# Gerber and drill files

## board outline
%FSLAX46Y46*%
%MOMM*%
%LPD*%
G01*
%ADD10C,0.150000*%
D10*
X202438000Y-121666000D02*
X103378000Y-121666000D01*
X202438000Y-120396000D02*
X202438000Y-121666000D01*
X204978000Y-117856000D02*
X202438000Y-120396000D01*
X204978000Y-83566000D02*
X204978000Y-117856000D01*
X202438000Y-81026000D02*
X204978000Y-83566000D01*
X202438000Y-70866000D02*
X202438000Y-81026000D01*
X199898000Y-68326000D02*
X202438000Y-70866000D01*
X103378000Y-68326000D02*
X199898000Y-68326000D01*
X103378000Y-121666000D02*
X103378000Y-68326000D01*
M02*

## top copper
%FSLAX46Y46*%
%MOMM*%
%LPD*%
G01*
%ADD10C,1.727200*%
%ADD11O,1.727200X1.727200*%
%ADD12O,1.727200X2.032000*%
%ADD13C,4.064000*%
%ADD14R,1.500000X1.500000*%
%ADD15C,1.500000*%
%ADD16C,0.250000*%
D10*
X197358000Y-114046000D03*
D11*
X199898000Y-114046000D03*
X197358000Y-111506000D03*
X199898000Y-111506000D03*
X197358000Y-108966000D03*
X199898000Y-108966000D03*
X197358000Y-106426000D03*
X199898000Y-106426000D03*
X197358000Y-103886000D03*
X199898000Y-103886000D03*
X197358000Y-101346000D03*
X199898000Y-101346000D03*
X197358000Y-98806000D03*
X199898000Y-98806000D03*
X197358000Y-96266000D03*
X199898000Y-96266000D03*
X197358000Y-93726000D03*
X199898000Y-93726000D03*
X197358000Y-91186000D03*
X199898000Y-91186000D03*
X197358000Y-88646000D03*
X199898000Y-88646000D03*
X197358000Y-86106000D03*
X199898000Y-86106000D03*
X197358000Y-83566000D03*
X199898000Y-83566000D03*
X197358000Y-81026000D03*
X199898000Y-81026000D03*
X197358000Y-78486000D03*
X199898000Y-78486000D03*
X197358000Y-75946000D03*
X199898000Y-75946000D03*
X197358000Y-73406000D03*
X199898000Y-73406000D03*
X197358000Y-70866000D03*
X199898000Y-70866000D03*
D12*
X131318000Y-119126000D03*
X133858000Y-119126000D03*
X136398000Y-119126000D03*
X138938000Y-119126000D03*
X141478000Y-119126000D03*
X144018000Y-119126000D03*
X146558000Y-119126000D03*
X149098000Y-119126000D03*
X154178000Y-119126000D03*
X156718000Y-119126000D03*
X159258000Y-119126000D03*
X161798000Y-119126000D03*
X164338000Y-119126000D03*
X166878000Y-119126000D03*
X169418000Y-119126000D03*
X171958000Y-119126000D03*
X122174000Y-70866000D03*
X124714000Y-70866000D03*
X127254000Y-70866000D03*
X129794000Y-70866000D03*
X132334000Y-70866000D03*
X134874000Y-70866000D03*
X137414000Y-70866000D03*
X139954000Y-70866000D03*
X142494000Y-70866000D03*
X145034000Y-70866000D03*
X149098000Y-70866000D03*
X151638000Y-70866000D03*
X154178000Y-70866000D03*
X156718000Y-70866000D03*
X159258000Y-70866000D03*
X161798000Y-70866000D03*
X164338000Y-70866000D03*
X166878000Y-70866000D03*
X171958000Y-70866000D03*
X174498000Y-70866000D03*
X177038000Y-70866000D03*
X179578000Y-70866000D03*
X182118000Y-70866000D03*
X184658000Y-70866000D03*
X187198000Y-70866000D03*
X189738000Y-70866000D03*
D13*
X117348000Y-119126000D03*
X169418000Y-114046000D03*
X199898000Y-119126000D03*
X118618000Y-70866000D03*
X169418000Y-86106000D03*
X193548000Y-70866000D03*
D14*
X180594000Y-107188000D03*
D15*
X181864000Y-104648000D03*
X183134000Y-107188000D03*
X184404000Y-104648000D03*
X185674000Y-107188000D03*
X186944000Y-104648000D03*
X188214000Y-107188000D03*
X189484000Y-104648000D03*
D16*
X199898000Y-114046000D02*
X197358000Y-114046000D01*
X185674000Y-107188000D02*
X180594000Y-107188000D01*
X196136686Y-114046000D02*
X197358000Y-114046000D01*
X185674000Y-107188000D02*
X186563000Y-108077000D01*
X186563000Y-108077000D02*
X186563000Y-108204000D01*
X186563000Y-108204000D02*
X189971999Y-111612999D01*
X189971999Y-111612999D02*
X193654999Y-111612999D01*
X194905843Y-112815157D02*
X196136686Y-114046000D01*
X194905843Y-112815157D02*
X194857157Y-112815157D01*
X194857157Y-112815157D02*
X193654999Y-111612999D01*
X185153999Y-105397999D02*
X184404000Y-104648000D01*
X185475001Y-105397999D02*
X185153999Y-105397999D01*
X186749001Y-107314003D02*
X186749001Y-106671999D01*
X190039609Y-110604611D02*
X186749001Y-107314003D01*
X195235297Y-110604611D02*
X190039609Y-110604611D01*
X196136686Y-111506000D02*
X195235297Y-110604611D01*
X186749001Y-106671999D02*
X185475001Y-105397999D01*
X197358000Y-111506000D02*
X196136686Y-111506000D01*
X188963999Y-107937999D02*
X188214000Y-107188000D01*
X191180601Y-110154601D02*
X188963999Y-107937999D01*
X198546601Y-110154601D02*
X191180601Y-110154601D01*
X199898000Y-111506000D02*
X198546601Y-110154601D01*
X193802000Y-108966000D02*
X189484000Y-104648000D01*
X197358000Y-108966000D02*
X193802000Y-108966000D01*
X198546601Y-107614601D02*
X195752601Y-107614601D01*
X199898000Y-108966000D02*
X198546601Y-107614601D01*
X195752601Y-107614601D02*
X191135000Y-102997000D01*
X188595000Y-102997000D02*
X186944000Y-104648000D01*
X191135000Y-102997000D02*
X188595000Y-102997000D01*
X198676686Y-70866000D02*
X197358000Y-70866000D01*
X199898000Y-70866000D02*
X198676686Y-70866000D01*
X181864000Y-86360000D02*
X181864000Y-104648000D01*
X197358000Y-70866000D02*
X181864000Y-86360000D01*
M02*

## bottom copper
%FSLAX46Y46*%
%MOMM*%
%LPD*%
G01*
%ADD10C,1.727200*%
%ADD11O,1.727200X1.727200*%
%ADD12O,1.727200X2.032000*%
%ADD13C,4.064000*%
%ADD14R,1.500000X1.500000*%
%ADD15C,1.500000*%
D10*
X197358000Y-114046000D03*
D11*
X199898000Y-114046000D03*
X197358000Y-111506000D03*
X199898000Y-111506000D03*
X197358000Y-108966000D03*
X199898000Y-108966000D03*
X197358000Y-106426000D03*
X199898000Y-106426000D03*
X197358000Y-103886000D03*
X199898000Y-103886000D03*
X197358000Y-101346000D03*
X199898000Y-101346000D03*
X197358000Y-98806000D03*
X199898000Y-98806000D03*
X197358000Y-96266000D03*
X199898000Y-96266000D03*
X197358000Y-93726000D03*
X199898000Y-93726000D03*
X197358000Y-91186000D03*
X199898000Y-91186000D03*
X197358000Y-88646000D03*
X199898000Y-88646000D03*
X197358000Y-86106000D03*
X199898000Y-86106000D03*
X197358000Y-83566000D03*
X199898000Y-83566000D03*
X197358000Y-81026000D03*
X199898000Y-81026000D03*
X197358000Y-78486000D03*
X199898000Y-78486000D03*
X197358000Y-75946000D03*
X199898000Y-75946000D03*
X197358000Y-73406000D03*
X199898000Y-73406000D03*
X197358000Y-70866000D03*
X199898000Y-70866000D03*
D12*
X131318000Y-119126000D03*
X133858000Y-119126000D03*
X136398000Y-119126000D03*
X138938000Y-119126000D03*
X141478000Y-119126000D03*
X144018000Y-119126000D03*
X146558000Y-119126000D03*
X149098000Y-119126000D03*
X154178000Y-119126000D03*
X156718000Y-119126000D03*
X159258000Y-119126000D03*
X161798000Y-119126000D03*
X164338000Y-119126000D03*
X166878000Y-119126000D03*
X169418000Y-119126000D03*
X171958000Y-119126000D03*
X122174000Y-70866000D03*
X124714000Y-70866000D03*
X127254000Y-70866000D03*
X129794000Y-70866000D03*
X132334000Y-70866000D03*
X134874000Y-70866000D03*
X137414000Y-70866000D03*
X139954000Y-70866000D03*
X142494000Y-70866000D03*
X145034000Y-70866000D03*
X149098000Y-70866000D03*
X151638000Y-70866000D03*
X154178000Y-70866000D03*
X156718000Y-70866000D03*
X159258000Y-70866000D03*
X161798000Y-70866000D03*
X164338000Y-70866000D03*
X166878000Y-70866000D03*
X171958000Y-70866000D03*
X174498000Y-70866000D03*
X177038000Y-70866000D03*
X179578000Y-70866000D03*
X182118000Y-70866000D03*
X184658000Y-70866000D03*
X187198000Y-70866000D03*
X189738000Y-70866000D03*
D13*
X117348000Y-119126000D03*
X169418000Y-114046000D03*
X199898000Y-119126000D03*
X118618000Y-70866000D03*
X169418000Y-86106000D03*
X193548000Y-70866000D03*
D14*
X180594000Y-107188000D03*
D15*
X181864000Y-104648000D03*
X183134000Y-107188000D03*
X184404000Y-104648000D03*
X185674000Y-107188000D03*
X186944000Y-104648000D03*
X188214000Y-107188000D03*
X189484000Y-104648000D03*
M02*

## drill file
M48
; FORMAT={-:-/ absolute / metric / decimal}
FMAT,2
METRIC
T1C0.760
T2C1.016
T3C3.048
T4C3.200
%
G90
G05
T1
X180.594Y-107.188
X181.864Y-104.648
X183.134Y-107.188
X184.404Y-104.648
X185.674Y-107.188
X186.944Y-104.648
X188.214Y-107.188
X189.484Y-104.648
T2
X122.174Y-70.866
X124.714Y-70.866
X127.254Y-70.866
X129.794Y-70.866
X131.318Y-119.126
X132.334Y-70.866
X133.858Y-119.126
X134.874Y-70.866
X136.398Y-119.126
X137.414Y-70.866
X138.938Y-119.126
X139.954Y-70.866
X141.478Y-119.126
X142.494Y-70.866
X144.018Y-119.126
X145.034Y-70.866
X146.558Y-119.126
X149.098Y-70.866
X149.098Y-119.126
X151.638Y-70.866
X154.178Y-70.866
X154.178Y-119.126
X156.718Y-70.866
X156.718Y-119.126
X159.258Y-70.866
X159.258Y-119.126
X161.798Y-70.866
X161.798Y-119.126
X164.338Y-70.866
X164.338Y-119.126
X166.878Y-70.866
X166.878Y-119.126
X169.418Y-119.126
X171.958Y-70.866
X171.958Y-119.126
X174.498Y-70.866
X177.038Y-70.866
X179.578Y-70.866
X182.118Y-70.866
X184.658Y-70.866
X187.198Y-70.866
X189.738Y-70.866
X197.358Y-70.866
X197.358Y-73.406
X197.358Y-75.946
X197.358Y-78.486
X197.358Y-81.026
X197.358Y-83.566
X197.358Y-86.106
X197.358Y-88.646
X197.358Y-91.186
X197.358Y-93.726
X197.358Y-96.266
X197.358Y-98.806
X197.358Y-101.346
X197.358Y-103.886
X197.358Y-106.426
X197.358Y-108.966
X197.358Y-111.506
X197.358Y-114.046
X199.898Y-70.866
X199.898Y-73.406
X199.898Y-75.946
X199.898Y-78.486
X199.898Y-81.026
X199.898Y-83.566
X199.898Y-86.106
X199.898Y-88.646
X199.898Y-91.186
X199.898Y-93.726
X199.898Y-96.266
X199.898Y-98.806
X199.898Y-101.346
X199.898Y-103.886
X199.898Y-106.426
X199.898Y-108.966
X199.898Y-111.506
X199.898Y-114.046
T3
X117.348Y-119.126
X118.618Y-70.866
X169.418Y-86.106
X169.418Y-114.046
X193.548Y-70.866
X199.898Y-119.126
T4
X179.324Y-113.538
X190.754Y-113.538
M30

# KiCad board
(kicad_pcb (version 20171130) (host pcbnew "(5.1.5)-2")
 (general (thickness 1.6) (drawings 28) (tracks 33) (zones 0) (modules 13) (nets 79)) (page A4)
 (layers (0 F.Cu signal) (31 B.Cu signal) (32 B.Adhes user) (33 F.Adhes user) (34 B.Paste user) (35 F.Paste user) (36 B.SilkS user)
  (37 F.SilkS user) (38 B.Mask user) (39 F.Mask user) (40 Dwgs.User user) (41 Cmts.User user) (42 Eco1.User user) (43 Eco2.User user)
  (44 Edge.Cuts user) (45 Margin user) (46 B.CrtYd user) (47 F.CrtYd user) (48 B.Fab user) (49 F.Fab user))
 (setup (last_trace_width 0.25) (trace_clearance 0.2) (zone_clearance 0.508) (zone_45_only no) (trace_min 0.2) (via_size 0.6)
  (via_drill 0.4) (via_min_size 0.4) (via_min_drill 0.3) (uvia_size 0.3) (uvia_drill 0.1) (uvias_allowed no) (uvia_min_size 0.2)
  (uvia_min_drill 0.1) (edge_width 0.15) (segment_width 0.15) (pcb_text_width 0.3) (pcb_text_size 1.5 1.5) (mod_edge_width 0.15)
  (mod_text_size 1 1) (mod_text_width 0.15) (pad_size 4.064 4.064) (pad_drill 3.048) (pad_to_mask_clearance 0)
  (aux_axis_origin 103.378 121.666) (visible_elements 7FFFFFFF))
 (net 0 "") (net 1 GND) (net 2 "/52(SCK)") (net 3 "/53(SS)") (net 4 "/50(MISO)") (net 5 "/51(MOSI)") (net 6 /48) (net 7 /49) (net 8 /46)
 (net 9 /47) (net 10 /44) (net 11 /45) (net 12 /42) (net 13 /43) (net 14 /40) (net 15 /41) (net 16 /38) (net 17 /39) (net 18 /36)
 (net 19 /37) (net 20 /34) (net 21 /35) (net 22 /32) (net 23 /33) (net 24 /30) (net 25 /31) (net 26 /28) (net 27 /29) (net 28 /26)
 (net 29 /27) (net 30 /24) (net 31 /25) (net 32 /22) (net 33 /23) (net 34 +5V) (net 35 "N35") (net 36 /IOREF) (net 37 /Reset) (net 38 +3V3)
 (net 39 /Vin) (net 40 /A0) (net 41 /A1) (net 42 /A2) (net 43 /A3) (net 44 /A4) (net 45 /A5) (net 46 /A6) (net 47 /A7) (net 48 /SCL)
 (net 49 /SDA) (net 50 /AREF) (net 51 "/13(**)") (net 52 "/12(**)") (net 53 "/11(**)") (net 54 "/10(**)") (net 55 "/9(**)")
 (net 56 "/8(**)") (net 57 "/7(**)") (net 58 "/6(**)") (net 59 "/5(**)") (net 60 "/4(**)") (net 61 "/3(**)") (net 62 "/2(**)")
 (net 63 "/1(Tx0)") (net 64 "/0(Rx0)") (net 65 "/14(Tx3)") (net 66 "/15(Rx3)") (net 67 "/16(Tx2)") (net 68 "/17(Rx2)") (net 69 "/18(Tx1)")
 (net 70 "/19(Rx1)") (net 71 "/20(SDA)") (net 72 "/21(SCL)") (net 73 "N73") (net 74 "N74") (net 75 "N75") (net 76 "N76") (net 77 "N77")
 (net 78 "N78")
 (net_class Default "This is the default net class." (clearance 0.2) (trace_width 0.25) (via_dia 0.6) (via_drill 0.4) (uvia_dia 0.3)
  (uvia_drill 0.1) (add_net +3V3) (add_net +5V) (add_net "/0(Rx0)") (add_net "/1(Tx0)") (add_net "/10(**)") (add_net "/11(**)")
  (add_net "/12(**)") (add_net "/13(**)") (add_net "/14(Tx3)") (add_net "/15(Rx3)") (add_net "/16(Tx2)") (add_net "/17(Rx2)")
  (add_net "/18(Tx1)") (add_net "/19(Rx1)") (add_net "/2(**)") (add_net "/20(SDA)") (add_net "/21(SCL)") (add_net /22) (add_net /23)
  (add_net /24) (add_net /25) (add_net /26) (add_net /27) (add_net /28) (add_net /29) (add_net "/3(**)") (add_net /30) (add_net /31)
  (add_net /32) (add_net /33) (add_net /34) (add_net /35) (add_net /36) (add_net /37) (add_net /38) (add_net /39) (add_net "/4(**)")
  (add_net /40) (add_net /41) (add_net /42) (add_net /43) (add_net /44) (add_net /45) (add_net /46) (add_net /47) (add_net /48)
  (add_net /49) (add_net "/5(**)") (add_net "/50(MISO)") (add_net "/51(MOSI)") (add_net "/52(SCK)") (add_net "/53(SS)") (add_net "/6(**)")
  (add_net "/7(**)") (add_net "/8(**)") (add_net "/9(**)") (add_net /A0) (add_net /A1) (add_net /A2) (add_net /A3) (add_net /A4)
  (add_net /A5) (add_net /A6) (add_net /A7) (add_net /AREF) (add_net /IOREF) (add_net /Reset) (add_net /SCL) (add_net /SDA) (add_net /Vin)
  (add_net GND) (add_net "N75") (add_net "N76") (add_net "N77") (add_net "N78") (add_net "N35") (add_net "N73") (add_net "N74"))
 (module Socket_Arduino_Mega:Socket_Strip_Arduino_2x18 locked (layer F.Cu) (at 197.358 114.046 90)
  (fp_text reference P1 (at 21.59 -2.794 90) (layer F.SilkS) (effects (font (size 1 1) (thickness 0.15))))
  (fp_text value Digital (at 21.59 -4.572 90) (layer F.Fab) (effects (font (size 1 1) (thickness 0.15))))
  (pad 1 thru_hole circle (at 0 0 90) (size 1.7272 1.7272) (drill 1.016) (layers *.Cu *.Mask F.SilkS) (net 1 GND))
  (pad 2 thru_hole oval (at 0 2.54 90) (size 1.7272 1.7272) (drill 1.016) (layers *.Cu *.Mask F.SilkS) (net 1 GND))
  (pad 3 thru_hole oval (at 2.54 0 90) (size 1.7272 1.7272) (drill 1.016) (layers *.Cu *.Mask F.SilkS) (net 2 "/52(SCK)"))
  (pad 4 thru_hole oval (at 2.54 2.54 90) (size 1.7272 1.7272) (drill 1.016) (layers *.Cu *.Mask F.SilkS) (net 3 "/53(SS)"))
  (pad 5 thru_hole oval (at 5.08 0 90) (size 1.7272 1.7272) (drill 1.016) (layers *.Cu *.Mask F.SilkS) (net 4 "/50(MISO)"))
  (pad 6 thru_hole oval (at 5.08 2.54 90) (size 1.7272 1.7272) (drill 1.016) (layers *.Cu *.Mask F.SilkS) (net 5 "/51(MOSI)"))
  (pad 7 thru_hole oval (at 7.62 0 90) (size 1.7272 1.7272) (drill 1.016) (layers *.Cu *.Mask F.SilkS) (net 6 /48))
  (pad 8 thru_hole oval (at 7.62 2.54 90) (size 1.7272 1.7272) (drill 1.016) (layers *.Cu *.Mask F.SilkS) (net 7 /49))
  (pad 9 thru_hole oval (at 10.16 0 90) (size 1.7272 1.7272) (drill 1.016) (layers *.Cu *.Mask F.SilkS) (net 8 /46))
  (pad 10 thru_hole oval (at 10.16 2.54 90) (size 1.7272 1.7272) (drill 1.016) (layers *.Cu *.Mask F.SilkS) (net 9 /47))
  (pad 11 thru_hole oval (at 12.7 0 90) (size 1.7272 1.7272) (drill 1.016) (layers *.Cu *.Mask F.SilkS) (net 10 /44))
  (pad 12 thru_hole oval (at 12.7 2.54 90) (size 1.7272 1.7272) (drill 1.016) (layers *.Cu *.Mask F.SilkS) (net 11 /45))
  (pad 13 thru_hole oval (at 15.24 0 90) (size 1.7272 1.7272) (drill 1.016) (layers *.Cu *.Mask F.SilkS) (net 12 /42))
  (pad 14 thru_hole oval (at 15.24 2.54 90) (size 1.7272 1.7272) (drill 1.016) (layers *.Cu *.Mask F.SilkS) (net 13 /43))
  (pad 15 thru_hole oval (at 17.78 0 90) (size 1.7272 1.7272) (drill 1.016) (layers *.Cu *.Mask F.SilkS) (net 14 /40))
  (pad 16 thru_hole oval (at 17.78 2.54 90) (size 1.7272 1.7272) (drill 1.016) (layers *.Cu *.Mask F.SilkS) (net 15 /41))
  (pad 17 thru_hole oval (at 20.32 0 90) (size 1.7272 1.7272) (drill 1.016) (layers *.Cu *.Mask F.SilkS) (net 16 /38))
  (pad 18 thru_hole oval (at 20.32 2.54 90) (size 1.7272 1.7272) (drill 1.016) (layers *.Cu *.Mask F.SilkS) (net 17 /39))
  (pad 19 thru_hole oval (at 22.86 0 90) (size 1.7272 1.7272) (drill 1.016) (layers *.Cu *.Mask F.SilkS) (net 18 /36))
  (pad 20 thru_hole oval (at 22.86 2.54 90) (size 1.7272 1.7272) (drill 1.016) (layers *.Cu *.Mask F.SilkS) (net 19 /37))
  (pad 21 thru_hole oval (at 25.4 0 90) (size 1.7272 1.7272) (drill 1.016) (layers *.Cu *.Mask F.SilkS) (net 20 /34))
  (pad 22 thru_hole oval (at 25.4 2.54 90) (size 1.7272 1.7272) (drill 1.016) (layers *.Cu *.Mask F.SilkS) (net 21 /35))
  (pad 23 thru_hole oval (at 27.94 0 90) (size 1.7272 1.7272) (drill 1.016) (layers *.Cu *.Mask F.SilkS) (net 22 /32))
  (pad 24 thru_hole oval (at 27.94 2.54 90) (size 1.7272 1.7272) (drill 1.016) (layers *.Cu *.Mask F.SilkS) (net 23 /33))
  (pad 25 thru_hole oval (at 30.48 0 90) (size 1.7272 1.7272) (drill 1.016) (layers *.Cu *.Mask F.SilkS) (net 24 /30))
  (pad 26 thru_hole oval (at 30.48 2.54 90) (size 1.7272 1.7272) (drill 1.016) (layers *.Cu *.Mask F.SilkS) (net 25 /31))
  (pad 27 thru_hole oval (at 33.02 0 90) (size 1.7272 1.7272) (drill 1.016) (layers *.Cu *.Mask F.SilkS) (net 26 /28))
  (pad 28 thru_hole oval (at 33.02 2.54 90) (size 1.7272 1.7272) (drill 1.016) (layers *.Cu *.Mask F.SilkS) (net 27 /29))
  (pad 29 thru_hole oval (at 35.56 0 90) (size 1.7272 1.7272) (drill 1.016) (layers *.Cu *.Mask F.SilkS) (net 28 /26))
  (pad 30 thru_hole oval (at 35.56 2.54 90) (size 1.7272 1.7272) (drill 1.016) (layers *.Cu *.Mask F.SilkS) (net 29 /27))
  (pad 31 thru_hole oval (at 38.1 0 90) (size 1.7272 1.7272) (drill 1.016) (layers *.Cu *.Mask F.SilkS) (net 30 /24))
  (pad 32 thru_hole oval (at 38.1 2.54 90) (size 1.7272 1.7272) (drill 1.016) (layers *.Cu *.Mask F.SilkS) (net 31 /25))
  (pad 33 thru_hole oval (at 40.64 0 90) (size 1.7272 1.7272) (drill 1.016) (layers *.Cu *.Mask F.SilkS) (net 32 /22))
  (pad 34 thru_hole oval (at 40.64 2.54 90) (size 1.7272 1.7272) (drill 1.016) (layers *.Cu *.Mask F.SilkS) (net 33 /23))
  (pad 35 thru_hole oval (at 43.18 0 90) (size 1.7272 1.7272) (drill 1.016) (layers *.Cu *.Mask F.SilkS) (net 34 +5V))
  (pad 36 thru_hole oval (at 43.18 2.54 90) (size 1.7272 1.7272) (drill 1.016) (layers *.Cu *.Mask F.SilkS) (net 34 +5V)))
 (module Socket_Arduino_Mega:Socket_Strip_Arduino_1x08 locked (layer F.Cu) (at 131.318 119.126)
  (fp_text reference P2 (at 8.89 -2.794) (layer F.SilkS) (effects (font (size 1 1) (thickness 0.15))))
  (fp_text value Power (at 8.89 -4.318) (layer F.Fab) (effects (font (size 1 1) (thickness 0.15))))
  (pad 1 thru_hole oval (at 0 0) (size 1.7272 2.032) (drill 1.016) (layers *.Cu *.Mask F.SilkS) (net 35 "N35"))
  (pad 2 thru_hole oval (at 2.54 0) (size 1.7272 2.032) (drill 1.016) (layers *.Cu *.Mask F.SilkS) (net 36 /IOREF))
  (pad 3 thru_hole oval (at 5.08 0) (size 1.7272 2.032) (drill 1.016) (layers *.Cu *.Mask F.SilkS) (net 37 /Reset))
  (pad 4 thru_hole oval (at 7.62 0) (size 1.7272 2.032) (drill 1.016) (layers *.Cu *.Mask F.SilkS) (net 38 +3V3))
  (pad 5 thru_hole oval (at 10.16 0) (size 1.7272 2.032) (drill 1.016) (layers *.Cu *.Mask F.SilkS) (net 34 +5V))
  (pad 6 thru_hole oval (at 12.7 0) (size 1.7272 2.032) (drill 1.016) (layers *.Cu *.Mask F.SilkS) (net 1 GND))
  (pad 7 thru_hole oval (at 15.24 0) (size 1.7272 2.032) (drill 1.016) (layers *.Cu *.Mask F.SilkS) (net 1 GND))
  (pad 8 thru_hole oval (at 17.78 0) (size 1.7272 2.032) (drill 1.016) (layers *.Cu *.Mask F.SilkS) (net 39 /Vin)))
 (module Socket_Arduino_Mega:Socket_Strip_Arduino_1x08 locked (layer F.Cu) (at 154.178 119.126)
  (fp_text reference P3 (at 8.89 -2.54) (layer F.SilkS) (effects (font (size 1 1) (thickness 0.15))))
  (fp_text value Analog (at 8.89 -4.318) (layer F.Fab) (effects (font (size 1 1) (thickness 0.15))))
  (pad 1 thru_hole oval (at 0 0) (size 1.7272 2.032) (drill 1.016) (layers *.Cu *.Mask F.SilkS) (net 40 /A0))
  (pad 2 thru_hole oval (at 2.54 0) (size 1.7272 2.032) (drill 1.016) (layers *.Cu *.Mask F.SilkS) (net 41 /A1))
  (pad 3 thru_hole oval (at 5.08 0) (size 1.7272 2.032) (drill 1.016) (layers *.Cu *.Mask F.SilkS) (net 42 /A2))
  (pad 4 thru_hole oval (at 7.62 0) (size 1.7272 2.032) (drill 1.016) (layers *.Cu *.Mask F.SilkS) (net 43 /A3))
  (pad 5 thru_hole oval (at 10.16 0) (size 1.7272 2.032) (drill 1.016) (layers *.Cu *.Mask F.SilkS) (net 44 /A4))
  (pad 6 thru_hole oval (at 12.7 0) (size 1.7272 2.032) (drill 1.016) (layers *.Cu *.Mask F.SilkS) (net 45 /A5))
  (pad 7 thru_hole oval (at 15.24 0) (size 1.7272 2.032) (drill 1.016) (layers *.Cu *.Mask F.SilkS) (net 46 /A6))
  (pad 8 thru_hole oval (at 17.78 0) (size 1.7272 2.032) (drill 1.016) (layers *.Cu *.Mask F.SilkS) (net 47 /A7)))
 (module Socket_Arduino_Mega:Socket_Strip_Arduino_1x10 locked (layer F.Cu) (at 122.174 70.866)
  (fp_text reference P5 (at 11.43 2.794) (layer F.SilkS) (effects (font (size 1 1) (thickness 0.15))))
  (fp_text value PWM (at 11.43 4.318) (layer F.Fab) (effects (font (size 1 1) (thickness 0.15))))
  (pad 1 thru_hole oval (at 0 0) (size 1.7272 2.032) (drill 1.016) (layers *.Cu *.Mask F.SilkS) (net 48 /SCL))
  (pad 2 thru_hole oval (at 2.54 0) (size 1.7272 2.032) (drill 1.016) (layers *.Cu *.Mask F.SilkS) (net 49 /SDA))
  (pad 3 thru_hole oval (at 5.08 0) (size 1.7272 2.032) (drill 1.016) (layers *.Cu *.Mask F.SilkS) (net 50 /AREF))
  (pad 4 thru_hole oval (at 7.62 0) (size 1.7272 2.032) (drill 1.016) (layers *.Cu *.Mask F.SilkS) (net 1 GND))
  (pad 5 thru_hole oval (at 10.16 0) (size 1.7272 2.032) (drill 1.016) (layers *.Cu *.Mask F.SilkS) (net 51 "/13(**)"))
  (pad 6 thru_hole oval (at 12.7 0) (size 1.7272 2.032) (drill 1.016) (layers *.Cu *.Mask F.SilkS) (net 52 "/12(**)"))
  (pad 7 thru_hole oval (at 15.24 0) (size 1.7272 2.032) (drill 1.016) (layers *.Cu *.Mask F.SilkS) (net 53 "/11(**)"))
  (pad 8 thru_hole oval (at 17.78 0) (size 1.7272 2.032) (drill 1.016) (layers *.Cu *.Mask F.SilkS) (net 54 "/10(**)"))
  (pad 9 thru_hole oval (at 20.32 0) (size 1.7272 2.032) (drill 1.016) (layers *.Cu *.Mask F.SilkS) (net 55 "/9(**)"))
  (pad 10 thru_hole oval (at 22.86 0) (size 1.7272 2.032) (drill 1.016) (layers *.Cu *.Mask F.SilkS) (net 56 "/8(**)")))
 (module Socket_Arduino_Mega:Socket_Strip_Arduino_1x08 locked (layer F.Cu) (at 149.098 70.866)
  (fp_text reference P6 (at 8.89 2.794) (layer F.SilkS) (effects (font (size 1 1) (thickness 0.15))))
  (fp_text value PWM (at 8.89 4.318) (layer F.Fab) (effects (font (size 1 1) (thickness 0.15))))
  (pad 1 thru_hole oval (at 0 0) (size 1.7272 2.032) (drill 1.016) (layers *.Cu *.Mask F.SilkS) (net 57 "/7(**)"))
  (pad 2 thru_hole oval (at 2.54 0) (size 1.7272 2.032) (drill 1.016) (layers *.Cu *.Mask F.SilkS) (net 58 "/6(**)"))
  (pad 3 thru_hole oval (at 5.08 0) (size 1.7272 2.032) (drill 1.016) (layers *.Cu *.Mask F.SilkS) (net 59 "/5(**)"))
  (pad 4 thru_hole oval (at 7.62 0) (size 1.7272 2.032) (drill 1.016) (layers *.Cu *.Mask F.SilkS) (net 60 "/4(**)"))
  (pad 5 thru_hole oval (at 10.16 0) (size 1.7272 2.032) (drill 1.016) (layers *.Cu *.Mask F.SilkS) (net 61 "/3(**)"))
  (pad 6 thru_hole oval (at 12.7 0) (size 1.7272 2.032) (drill 1.016) (layers *.Cu *.Mask F.SilkS) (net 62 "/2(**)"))
  (pad 7 thru_hole oval (at 15.24 0) (size 1.7272 2.032) (drill 1.016) (layers *.Cu *.Mask F.SilkS) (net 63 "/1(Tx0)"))
  (pad 8 thru_hole oval (at 17.78 0) (size 1.7272 2.032) (drill 1.016) (layers *.Cu *.Mask F.SilkS) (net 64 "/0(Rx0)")))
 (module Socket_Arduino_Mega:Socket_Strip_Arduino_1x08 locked (layer F.Cu) (at 171.958 70.866)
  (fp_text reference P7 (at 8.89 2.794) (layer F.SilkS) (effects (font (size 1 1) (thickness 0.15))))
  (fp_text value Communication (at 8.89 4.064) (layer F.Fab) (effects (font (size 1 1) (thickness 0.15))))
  (pad 1 thru_hole oval (at 0 0) (size 1.7272 2.032) (drill 1.016) (layers *.Cu *.Mask F.SilkS) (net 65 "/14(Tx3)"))
  (pad 2 thru_hole oval (at 2.54 0) (size 1.7272 2.032) (drill 1.016) (layers *.Cu *.Mask F.SilkS) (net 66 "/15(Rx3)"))
  (pad 3 thru_hole oval (at 5.08 0) (size 1.7272 2.032) (drill 1.016) (layers *.Cu *.Mask F.SilkS) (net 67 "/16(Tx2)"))
  (pad 4 thru_hole oval (at 7.62 0) (size 1.7272 2.032) (drill 1.016) (layers *.Cu *.Mask F.SilkS) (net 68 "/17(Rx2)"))
  (pad 5 thru_hole oval (at 10.16 0) (size 1.7272 2.032) (drill 1.016) (layers *.Cu *.Mask F.SilkS) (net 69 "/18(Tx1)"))
  (pad 6 thru_hole oval (at 12.7 0) (size 1.7272 2.032) (drill 1.016) (layers *.Cu *.Mask F.SilkS) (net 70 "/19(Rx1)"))
  (pad 7 thru_hole oval (at 15.24 0) (size 1.7272 2.032) (drill 1.016) (layers *.Cu *.Mask F.SilkS) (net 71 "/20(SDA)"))
  (pad 8 thru_hole oval (at 17.78 0) (size 1.7272 2.032) (drill 1.016) (layers *.Cu *.Mask F.SilkS) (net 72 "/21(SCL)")))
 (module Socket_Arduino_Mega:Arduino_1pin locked (layer F.Cu) (at 117.348 119.126)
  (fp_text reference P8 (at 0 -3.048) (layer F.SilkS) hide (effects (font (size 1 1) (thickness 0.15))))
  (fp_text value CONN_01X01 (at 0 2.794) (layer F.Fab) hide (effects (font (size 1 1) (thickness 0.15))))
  (pad 1 thru_hole circle (at 0 0) (size 4.064 4.064) (drill 3.048) (layers *.Cu *.Mask F.SilkS) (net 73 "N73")))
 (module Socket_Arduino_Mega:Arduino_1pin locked (layer F.Cu) (at 169.418 114.046)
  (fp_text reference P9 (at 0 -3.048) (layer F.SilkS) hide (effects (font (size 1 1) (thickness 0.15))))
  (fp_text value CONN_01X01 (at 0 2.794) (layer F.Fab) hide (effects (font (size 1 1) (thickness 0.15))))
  (pad 1 thru_hole circle (at 0 0) (size 4.064 4.064) (drill 3.048) (layers *.Cu *.Mask F.SilkS) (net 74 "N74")))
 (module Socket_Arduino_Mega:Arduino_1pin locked (layer F.Cu) (at 199.898 119.126)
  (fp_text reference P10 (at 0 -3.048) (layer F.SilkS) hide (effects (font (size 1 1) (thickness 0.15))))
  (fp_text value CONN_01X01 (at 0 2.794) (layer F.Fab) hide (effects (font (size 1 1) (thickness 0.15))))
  (pad 1 thru_hole circle (at 0 0) (size 4.064 4.064) (drill 3.048) (layers *.Cu *.Mask F.SilkS) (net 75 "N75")))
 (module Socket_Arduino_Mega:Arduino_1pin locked (layer F.Cu) (at 118.618 70.866)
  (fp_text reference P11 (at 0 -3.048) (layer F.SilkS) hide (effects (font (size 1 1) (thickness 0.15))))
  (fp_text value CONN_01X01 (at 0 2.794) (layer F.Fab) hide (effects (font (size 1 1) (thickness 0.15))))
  (pad 1 thru_hole circle (at 0 0) (size 4.064 4.064) (drill 3.048) (layers *.Cu *.Mask F.SilkS) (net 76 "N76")))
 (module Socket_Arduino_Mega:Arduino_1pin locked (layer F.Cu) (at 169.418 86.106)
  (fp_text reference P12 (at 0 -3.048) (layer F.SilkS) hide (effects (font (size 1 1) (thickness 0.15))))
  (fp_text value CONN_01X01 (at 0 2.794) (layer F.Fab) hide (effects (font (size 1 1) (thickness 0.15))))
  (pad 1 thru_hole circle (at 0 0) (size 4.064 4.064) (drill 3.048) (layers *.Cu *.Mask F.SilkS) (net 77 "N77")))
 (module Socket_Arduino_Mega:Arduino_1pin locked (layer F.Cu) (at 193.548 70.866)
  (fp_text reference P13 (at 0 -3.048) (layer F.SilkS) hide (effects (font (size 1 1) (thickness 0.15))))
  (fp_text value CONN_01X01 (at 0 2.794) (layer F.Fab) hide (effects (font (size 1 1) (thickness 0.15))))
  (pad 1 thru_hole circle (at 0 0) (size 4.064 4.064) (drill 3.048) (layers *.Cu *.Mask F.SilkS) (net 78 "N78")))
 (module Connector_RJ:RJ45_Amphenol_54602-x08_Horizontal (layer F.Cu) (at 180.594 107.188)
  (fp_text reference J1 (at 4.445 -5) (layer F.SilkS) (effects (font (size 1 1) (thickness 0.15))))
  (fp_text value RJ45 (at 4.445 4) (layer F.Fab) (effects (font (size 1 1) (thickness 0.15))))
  (pad "" np_thru_hole circle (at 10.16 6.35) (size 3.2 3.2) (drill 3.2) (layers *.Cu *.Mask))
  (pad "" np_thru_hole circle (at -1.27 6.35) (size 3.2 3.2) (drill 3.2) (layers *.Cu *.Mask))
  (pad 1 thru_hole rect (at 0 0) (size 1.5 1.5) (drill 0.76) (layers *.Cu *.Mask) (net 1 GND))
  (pad 2 thru_hole circle (at 1.27 -2.54) (size 1.5 1.5) (drill 0.76) (layers *.Cu *.Mask) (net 34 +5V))
  (pad 3 thru_hole circle (at 2.54 0) (size 1.5 1.5) (drill 0.76) (layers *.Cu *.Mask) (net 1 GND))
  (pad 4 thru_hole circle (at 3.81 -2.54) (size 1.5 1.5) (drill 0.76) (layers *.Cu *.Mask) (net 2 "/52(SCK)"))
  (pad 5 thru_hole circle (at 5.08 0) (size 1.5 1.5) (drill 0.76) (layers *.Cu *.Mask) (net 1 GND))
  (pad 6 thru_hole circle (at 6.35 -2.54) (size 1.5 1.5) (drill 0.76) (layers *.Cu *.Mask) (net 5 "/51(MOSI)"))
  (pad 7 thru_hole circle (at 7.62 0) (size 1.5 1.5) (drill 0.76) (layers *.Cu *.Mask) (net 3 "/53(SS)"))
  (pad 8 thru_hole circle (at 8.89 -2.54) (size 1.5 1.5) (drill 0.76) (layers *.Cu *.Mask) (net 4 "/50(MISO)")))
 (gr_line (start 202.438 121.666) (end 103.378 121.666) (angle 90) (layer Edge.Cuts) (width 0.15))
 (gr_line (start 202.438 120.396) (end 202.438 121.666) (angle 90) (layer Edge.Cuts) (width 0.15))
 (gr_line (start 204.978 117.856) (end 202.438 120.396) (angle 90) (layer Edge.Cuts) (width 0.15))
 (gr_line (start 204.978 83.566) (end 204.978 117.856) (angle 90) (layer Edge.Cuts) (width 0.15))
 (gr_line (start 202.438 81.026) (end 204.978 83.566) (angle 90) (layer Edge.Cuts) (width 0.15))
 (gr_line (start 202.438 70.866) (end 202.438 81.026) (angle 90) (layer Edge.Cuts) (width 0.15))
 (gr_line (start 199.898 68.326) (end 202.438 70.866) (angle 90) (layer Edge.Cuts) (width 0.15))
 (gr_line (start 103.378 68.326) (end 199.898 68.326) (angle 90) (layer Edge.Cuts) (width 0.15))
 (gr_line (start 103.378 121.666) (end 103.378 68.326) (angle 90) (layer Edge.Cuts) (width 0.15))
 (segment (start 199.898 114.046) (end 197.358 114.046) (width 0.25) (layer F.Cu) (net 1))
 (segment (start 185.674 107.188) (end 180.594 107.188) (width 0.25) (layer F.Cu) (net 1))
 (segment (start 196.136686 114.046) (end 197.358 114.046) (width 0.25) (layer F.Cu) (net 1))
 (segment (start 185.674 107.188) (end 186.563 108.077) (width 0.25) (layer F.Cu) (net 1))
 (segment (start 186.563 108.077) (end 186.563 108.204) (width 0.25) (layer F.Cu) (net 1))
 (segment (start 186.563 108.204) (end 189.971999 111.612999) (width 0.25) (layer F.Cu) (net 1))
 (segment (start 189.971999 111.612999) (end 193.654999 111.612999) (width 0.25) (layer F.Cu) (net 1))
 (segment (start 194.905843 112.815157) (end 196.136686 114.046) (width 0.25) (layer F.Cu) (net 1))
 (segment (start 194.905843 112.815157) (end 194.857157 112.815157) (width 0.25) (layer F.Cu) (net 1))
 (segment (start 194.857157 112.815157) (end 193.654999 111.612999) (width 0.25) (layer F.Cu) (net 1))
 (segment (start 185.153999 105.397999) (end 184.404 104.648) (width 0.25) (layer F.Cu) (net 2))
 (segment (start 185.475001 105.397999) (end 185.153999 105.397999) (width 0.25) (layer F.Cu) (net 2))
 (segment (start 186.749001 107.314003) (end 186.749001 106.671999) (width 0.25) (layer F.Cu) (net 2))
 (segment (start 190.039609 110.604611) (end 186.749001 107.314003) (width 0.25) (layer F.Cu) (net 2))
 (segment (start 195.235297 110.604611) (end 190.039609 110.604611) (width 0.25) (layer F.Cu) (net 2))
 (segment (start 196.136686 111.506) (end 195.235297 110.604611) (width 0.25) (layer F.Cu) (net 2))
 (segment (start 186.749001 106.671999) (end 185.475001 105.397999) (width 0.25) (layer F.Cu) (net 2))
 (segment (start 197.358 111.506) (end 196.136686 111.506) (width 0.25) (layer F.Cu) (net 2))
 (segment (start 188.963999 107.937999) (end 188.214 107.188) (width 0.25) (layer F.Cu) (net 3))
 (segment (start 191.180601 110.154601) (end 188.963999 107.937999) (width 0.25) (layer F.Cu) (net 3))
 (segment (start 198.546601 110.154601) (end 191.180601 110.154601) (width 0.25) (layer F.Cu) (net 3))
 (segment (start 199.898 111.506) (end 198.546601 110.154601) (width 0.25) (layer F.Cu) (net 3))
 (segment (start 193.802 108.966) (end 189.484 104.648) (width 0.25) (layer F.Cu) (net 4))
 (segment (start 197.358 108.966) (end 193.802 108.966) (width 0.25) (layer F.Cu) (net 4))
 (segment (start 198.546601 107.614601) (end 195.752601 107.614601) (width 0.25) (layer F.Cu) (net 5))
 (segment (start 199.898 108.966) (end 198.546601 107.614601) (width 0.25) (layer F.Cu) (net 5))
 (segment (start 195.752601 107.614601) (end 191.135 102.997) (width 0.25) (layer F.Cu) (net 5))
 (segment (start 188.595 102.997) (end 186.944 104.648) (width 0.25) (layer F.Cu) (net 5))
 (segment (start 191.135 102.997) (end 188.595 102.997) (width 0.25) (layer F.Cu) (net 5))
 (segment (start 198.676686 70.866) (end 197.358 70.866) (width 0.25) (layer F.Cu) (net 34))
 (segment (start 199.898 70.866) (end 198.676686 70.866) (width 0.25) (layer F.Cu) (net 34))
 (segment (start 181.864 86.36) (end 181.864 104.648) (width 0.25) (layer F.Cu) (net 34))
 (segment (start 197.358 70.866) (end 181.864 86.36) (width 0.25) (layer F.Cu) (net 34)))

